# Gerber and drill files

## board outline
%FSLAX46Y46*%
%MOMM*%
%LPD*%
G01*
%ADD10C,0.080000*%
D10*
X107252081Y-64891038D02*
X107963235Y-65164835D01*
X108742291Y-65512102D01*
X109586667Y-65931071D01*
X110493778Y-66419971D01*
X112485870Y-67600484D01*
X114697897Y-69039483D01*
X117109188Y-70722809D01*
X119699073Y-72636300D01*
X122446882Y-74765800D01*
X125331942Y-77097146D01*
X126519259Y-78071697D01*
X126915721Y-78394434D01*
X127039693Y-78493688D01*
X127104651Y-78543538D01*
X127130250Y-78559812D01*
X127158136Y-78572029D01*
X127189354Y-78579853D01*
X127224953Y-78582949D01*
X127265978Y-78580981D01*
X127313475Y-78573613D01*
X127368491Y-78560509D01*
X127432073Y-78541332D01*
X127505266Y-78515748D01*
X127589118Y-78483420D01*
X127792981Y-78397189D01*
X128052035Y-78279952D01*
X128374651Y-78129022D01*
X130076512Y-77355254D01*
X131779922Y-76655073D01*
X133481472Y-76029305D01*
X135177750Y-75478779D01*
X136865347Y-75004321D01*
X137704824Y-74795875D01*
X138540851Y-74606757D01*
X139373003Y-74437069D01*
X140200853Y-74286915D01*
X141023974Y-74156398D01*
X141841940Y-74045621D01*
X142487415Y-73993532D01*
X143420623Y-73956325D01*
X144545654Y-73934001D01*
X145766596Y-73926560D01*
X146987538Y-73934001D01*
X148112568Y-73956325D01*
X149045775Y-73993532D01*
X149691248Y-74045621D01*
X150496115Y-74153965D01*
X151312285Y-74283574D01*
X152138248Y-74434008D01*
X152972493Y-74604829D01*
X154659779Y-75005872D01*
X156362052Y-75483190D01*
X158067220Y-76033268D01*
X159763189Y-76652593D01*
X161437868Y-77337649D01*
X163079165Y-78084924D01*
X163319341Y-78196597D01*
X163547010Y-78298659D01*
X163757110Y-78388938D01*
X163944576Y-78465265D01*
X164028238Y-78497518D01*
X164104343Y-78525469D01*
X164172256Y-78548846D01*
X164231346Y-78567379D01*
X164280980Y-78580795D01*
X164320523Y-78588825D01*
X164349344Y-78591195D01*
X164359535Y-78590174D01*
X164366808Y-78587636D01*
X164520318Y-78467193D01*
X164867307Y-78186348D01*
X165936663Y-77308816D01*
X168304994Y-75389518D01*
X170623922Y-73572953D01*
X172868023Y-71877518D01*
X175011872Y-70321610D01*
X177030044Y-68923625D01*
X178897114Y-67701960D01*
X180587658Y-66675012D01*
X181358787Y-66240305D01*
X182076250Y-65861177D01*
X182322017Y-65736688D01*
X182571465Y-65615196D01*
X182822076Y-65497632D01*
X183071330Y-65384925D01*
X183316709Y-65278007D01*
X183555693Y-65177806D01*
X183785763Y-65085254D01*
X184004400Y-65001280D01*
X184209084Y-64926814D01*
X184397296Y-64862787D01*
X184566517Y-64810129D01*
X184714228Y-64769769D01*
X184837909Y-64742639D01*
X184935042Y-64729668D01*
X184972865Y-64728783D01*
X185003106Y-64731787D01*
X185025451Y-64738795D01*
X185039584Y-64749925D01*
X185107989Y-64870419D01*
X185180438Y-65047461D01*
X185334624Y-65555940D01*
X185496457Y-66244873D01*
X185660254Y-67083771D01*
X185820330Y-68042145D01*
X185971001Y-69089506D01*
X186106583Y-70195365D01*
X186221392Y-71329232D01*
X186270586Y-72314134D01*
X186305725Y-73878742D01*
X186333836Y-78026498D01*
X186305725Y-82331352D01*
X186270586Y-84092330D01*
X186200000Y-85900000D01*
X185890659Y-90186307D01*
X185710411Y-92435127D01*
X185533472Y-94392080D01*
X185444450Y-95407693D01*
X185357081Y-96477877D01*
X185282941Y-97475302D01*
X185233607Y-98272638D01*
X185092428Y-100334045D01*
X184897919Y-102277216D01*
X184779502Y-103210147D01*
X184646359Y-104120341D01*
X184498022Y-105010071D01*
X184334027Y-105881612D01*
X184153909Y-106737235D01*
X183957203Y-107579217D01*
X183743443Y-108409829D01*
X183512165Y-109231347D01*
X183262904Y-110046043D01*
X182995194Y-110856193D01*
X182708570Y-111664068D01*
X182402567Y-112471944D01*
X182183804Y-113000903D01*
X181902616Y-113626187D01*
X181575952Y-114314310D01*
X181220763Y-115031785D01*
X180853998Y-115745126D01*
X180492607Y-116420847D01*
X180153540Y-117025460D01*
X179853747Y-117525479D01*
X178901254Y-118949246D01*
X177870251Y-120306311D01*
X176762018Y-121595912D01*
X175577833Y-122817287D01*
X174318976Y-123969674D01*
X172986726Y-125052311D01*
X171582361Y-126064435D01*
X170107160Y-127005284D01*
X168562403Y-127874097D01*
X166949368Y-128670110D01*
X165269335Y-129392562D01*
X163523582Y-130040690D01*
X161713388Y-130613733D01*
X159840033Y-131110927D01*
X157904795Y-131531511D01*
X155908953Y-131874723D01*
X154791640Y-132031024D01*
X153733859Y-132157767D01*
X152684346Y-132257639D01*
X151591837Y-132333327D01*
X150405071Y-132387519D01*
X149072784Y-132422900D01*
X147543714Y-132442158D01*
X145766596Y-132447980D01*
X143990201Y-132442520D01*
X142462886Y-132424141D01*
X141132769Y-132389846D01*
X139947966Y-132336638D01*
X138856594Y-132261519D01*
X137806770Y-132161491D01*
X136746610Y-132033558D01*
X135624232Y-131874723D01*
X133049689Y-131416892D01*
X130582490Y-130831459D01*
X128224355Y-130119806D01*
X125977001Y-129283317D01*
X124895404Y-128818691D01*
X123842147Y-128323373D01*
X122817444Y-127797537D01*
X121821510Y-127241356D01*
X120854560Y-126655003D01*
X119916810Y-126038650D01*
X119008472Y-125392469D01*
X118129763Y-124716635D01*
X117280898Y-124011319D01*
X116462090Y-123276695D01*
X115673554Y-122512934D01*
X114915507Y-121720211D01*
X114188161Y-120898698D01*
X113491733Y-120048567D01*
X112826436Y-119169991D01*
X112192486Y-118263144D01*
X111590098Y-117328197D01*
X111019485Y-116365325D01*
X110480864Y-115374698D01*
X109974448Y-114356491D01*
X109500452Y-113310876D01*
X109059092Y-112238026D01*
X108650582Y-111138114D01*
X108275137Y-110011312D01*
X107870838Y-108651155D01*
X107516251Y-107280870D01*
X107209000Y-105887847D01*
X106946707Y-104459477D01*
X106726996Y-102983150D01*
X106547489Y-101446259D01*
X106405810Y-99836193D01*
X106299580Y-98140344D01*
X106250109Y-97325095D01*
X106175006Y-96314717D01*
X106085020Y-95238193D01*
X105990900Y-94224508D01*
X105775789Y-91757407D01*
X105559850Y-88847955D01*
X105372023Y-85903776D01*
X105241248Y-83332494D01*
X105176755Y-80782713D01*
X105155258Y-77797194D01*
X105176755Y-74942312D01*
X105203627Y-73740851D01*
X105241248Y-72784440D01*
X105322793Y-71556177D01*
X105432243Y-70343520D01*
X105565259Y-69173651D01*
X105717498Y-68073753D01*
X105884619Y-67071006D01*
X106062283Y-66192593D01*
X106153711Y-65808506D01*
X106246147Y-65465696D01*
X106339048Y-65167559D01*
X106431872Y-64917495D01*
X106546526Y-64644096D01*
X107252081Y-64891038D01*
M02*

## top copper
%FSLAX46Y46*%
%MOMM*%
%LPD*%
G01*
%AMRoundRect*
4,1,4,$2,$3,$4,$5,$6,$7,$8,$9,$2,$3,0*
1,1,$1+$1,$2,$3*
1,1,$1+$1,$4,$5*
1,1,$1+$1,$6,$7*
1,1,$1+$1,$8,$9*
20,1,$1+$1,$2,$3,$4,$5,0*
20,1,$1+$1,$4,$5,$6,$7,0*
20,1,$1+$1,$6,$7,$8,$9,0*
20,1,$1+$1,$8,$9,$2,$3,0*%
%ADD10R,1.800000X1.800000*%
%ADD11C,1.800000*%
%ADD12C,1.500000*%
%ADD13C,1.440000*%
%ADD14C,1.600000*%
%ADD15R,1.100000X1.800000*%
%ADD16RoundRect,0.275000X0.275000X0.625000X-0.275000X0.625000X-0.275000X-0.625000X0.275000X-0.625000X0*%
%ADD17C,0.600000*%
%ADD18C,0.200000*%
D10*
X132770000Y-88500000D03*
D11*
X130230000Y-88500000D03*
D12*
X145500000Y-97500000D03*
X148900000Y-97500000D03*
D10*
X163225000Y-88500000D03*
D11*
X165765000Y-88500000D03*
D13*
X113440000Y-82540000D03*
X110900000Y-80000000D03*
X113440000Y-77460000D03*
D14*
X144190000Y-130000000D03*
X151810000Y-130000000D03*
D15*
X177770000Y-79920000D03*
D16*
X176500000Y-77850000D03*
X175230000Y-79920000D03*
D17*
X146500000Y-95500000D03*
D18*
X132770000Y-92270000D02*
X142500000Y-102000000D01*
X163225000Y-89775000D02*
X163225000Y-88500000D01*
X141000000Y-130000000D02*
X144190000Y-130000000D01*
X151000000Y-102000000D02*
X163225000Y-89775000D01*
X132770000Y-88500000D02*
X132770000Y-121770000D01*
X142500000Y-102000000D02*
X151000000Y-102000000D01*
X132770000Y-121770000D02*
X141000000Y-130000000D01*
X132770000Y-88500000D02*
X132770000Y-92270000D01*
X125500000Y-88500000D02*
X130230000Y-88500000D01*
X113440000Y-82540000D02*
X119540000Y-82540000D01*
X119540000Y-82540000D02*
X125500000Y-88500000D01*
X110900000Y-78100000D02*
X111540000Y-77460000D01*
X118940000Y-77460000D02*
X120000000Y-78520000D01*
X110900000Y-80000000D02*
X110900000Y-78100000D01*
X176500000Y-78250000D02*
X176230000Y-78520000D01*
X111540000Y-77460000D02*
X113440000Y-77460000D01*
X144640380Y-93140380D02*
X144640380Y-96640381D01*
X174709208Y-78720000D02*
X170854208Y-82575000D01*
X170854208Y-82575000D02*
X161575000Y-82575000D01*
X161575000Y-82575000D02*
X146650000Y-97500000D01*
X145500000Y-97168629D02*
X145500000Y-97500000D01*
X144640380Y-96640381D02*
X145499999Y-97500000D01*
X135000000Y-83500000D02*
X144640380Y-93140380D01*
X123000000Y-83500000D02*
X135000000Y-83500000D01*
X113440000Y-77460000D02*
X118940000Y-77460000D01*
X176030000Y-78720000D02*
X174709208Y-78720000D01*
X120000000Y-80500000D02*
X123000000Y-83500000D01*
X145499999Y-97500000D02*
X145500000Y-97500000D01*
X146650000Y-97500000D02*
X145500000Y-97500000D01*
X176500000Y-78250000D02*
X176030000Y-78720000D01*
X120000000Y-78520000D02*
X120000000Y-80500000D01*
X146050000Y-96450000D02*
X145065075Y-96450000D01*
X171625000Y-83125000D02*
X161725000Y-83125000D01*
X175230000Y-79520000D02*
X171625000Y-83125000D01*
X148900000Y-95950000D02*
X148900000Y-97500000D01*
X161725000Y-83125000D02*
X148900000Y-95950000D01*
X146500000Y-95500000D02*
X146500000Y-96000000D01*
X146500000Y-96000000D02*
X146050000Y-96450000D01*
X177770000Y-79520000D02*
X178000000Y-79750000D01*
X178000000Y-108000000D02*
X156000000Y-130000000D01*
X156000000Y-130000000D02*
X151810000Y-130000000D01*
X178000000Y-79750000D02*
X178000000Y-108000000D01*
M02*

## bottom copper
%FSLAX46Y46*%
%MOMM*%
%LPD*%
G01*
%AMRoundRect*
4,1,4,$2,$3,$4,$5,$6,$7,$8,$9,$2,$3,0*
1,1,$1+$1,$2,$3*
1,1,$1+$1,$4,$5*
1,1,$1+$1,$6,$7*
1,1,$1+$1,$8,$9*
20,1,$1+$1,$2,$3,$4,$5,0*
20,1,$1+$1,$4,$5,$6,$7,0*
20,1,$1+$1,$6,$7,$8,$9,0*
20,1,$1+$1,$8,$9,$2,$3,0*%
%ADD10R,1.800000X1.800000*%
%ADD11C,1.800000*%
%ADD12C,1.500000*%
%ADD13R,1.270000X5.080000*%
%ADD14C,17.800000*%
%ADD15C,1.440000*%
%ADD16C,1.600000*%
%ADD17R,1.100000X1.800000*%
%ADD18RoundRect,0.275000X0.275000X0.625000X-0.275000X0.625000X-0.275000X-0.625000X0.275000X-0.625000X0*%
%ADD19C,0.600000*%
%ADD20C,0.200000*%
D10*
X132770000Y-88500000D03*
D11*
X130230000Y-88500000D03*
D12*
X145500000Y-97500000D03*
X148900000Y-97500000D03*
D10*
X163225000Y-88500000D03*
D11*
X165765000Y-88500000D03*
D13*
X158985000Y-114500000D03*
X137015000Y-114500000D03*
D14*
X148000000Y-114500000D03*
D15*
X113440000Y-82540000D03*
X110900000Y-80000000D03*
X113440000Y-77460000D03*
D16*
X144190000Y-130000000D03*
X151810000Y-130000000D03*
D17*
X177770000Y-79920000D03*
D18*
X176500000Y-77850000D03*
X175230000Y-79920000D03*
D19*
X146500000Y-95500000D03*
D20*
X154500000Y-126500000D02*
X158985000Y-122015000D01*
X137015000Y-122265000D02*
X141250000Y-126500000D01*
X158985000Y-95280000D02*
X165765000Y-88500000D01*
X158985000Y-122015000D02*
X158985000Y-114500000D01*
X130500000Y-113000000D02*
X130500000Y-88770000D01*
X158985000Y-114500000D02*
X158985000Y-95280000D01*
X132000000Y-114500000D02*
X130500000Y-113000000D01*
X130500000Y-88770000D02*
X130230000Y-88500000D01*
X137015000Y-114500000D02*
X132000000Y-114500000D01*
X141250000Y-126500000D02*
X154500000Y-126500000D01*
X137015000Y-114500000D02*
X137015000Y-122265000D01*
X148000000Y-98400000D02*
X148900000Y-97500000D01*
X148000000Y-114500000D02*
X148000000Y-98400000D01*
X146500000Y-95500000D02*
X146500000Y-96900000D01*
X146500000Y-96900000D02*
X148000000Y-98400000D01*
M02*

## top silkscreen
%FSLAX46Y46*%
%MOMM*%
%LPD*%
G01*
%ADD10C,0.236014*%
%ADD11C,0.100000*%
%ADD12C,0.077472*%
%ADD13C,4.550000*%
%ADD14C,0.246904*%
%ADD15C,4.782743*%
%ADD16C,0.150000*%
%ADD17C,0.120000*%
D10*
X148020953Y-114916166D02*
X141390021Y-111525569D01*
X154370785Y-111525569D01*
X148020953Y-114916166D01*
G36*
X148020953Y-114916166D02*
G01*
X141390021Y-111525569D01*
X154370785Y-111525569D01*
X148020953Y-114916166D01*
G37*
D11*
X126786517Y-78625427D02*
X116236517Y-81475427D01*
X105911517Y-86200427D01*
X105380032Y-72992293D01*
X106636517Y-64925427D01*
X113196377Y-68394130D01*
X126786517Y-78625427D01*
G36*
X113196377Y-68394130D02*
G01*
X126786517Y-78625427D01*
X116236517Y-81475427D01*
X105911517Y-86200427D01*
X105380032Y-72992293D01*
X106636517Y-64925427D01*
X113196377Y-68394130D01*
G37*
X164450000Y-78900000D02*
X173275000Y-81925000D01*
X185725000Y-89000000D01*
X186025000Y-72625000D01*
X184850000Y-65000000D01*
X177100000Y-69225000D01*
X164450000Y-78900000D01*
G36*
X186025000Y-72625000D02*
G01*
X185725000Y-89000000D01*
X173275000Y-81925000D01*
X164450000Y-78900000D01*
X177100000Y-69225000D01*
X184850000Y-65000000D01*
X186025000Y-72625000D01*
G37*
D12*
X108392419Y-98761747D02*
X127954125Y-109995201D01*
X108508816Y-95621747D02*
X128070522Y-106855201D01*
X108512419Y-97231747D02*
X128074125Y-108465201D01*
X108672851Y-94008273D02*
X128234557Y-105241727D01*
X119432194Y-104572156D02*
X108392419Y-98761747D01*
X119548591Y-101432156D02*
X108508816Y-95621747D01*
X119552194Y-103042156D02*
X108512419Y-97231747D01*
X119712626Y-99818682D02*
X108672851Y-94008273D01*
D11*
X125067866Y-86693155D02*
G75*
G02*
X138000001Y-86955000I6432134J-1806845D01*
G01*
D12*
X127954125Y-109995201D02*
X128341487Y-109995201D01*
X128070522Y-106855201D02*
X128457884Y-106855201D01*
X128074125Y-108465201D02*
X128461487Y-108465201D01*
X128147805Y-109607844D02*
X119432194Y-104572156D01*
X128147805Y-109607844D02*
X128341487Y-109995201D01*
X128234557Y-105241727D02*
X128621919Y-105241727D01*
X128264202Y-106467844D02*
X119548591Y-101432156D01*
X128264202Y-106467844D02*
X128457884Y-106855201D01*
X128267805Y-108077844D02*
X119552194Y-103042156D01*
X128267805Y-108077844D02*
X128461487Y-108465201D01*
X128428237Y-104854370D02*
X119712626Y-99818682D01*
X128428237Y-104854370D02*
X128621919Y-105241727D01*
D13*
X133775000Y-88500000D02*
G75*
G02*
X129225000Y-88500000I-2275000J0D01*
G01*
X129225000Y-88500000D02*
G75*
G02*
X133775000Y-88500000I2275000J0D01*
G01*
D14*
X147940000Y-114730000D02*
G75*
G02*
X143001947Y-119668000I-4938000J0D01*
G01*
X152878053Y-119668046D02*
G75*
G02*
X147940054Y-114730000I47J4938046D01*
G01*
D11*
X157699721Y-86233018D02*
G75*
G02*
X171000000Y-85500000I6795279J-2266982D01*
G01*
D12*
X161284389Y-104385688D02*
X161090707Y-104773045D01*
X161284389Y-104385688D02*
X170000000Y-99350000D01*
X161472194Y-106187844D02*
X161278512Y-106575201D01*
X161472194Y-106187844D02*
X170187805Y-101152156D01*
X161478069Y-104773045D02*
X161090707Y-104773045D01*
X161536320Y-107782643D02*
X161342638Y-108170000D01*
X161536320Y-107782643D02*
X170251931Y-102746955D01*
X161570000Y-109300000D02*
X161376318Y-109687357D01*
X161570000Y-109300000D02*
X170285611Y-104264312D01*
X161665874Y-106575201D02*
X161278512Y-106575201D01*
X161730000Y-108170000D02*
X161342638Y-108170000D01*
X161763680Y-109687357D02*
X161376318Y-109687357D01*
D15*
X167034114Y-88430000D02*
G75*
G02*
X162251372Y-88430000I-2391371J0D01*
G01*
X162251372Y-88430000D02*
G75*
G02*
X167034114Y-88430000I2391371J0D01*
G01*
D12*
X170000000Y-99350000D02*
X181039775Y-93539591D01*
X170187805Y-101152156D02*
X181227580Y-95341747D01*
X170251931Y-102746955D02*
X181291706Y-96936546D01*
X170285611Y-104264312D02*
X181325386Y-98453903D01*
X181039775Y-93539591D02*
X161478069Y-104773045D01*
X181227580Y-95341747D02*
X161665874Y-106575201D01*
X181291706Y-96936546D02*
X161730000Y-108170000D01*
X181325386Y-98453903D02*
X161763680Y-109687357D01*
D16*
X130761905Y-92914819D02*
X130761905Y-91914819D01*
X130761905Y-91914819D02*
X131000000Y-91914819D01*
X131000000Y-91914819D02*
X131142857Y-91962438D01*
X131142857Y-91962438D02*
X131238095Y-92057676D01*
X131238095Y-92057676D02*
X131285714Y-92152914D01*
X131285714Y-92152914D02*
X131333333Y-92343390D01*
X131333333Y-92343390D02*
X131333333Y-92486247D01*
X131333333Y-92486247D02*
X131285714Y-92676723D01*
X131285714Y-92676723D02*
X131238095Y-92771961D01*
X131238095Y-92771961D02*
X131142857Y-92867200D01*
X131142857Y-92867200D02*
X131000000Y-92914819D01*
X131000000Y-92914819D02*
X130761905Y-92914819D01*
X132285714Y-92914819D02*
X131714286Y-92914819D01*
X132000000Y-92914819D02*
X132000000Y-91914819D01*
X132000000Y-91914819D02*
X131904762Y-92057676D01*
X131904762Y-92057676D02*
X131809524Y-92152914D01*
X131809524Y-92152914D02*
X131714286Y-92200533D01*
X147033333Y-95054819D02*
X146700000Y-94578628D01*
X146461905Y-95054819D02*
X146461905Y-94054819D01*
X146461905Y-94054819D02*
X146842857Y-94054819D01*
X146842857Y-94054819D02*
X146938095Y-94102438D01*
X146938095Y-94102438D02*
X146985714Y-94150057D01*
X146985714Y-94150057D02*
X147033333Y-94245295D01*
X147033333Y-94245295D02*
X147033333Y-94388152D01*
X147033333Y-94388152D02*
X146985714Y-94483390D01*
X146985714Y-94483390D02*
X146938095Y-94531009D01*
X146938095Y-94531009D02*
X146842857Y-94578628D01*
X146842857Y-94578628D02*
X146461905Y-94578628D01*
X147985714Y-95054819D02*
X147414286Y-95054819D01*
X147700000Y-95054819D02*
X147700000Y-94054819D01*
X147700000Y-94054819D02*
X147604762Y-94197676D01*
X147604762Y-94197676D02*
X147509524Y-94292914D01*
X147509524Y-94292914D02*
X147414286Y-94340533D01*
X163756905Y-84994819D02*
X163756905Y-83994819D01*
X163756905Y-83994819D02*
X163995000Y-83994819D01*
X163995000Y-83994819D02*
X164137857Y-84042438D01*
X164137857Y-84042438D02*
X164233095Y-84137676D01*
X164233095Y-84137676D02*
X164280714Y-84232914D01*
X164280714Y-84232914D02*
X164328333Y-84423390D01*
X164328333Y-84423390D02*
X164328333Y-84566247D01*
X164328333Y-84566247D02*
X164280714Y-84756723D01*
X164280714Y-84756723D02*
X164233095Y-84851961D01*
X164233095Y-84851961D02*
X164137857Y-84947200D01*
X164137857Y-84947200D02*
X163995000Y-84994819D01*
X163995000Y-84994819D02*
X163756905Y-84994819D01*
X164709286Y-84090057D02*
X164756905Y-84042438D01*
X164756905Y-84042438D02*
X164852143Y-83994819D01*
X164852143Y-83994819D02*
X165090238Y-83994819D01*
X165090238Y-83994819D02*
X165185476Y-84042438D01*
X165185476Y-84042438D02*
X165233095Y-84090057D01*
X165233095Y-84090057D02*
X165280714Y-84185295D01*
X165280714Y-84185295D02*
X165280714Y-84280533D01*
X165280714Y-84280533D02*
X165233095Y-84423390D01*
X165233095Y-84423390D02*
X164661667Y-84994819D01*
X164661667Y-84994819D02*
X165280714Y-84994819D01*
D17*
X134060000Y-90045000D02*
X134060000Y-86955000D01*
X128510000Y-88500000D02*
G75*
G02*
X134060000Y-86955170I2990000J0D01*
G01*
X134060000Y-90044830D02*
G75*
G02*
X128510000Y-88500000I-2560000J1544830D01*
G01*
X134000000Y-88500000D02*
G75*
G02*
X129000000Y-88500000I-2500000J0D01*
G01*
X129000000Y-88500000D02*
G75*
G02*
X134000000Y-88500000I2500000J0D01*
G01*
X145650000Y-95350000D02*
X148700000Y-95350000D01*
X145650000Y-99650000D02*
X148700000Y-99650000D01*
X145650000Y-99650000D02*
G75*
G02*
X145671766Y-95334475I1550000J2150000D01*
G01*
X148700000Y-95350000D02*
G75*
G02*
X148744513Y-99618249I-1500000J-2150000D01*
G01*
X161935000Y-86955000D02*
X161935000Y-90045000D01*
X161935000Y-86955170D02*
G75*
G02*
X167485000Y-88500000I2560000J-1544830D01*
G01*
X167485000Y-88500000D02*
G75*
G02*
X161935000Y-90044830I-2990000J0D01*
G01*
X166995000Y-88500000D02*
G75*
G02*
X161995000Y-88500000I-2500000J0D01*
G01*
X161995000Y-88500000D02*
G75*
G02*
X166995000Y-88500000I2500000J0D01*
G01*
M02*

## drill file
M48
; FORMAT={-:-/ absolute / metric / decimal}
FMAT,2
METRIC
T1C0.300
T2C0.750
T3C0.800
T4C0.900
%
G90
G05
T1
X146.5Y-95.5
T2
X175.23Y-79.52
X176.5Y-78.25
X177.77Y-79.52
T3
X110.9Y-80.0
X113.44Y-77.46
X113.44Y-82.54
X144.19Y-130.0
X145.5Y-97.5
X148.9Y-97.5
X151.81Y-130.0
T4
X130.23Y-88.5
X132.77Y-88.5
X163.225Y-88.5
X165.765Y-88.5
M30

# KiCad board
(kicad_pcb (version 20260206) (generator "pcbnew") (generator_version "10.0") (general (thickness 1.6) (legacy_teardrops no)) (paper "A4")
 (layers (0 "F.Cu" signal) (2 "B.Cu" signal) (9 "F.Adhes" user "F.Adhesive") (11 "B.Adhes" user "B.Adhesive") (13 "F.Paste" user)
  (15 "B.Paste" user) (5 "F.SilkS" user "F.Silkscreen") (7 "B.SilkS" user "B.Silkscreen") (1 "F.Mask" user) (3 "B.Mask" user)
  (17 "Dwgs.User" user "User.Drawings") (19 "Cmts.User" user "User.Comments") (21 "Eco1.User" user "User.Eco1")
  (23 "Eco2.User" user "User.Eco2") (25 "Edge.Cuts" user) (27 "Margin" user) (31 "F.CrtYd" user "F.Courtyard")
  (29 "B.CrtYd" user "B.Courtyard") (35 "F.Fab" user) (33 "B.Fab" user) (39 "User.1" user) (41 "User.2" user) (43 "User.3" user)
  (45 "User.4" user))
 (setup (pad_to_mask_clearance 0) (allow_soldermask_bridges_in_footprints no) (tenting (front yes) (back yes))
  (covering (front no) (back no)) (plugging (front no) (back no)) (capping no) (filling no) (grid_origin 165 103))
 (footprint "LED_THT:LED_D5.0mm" (layer "F.Cu") (at 132.77 88.5 180)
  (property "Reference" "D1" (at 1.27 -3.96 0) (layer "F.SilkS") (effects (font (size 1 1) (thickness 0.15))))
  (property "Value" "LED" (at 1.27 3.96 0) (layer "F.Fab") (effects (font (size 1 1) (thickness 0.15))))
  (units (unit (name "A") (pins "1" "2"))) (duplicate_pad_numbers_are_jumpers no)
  (fp_line (start -1.29 -1.545) (end -1.29 1.545) (stroke (width 0.12) (type solid)) (layer "F.SilkS"))
  (fp_arc (start 4.26 0) (mid 2.071779 2.880495) (end -1.29 1.54483) (stroke (width 0.12) (type solid)) (layer "F.SilkS"))
  (fp_arc (start -1.29 -1.54483) (mid 2.071779 -2.880495) (end 4.26 0) (stroke (width 0.12) (type solid)) (layer "F.SilkS"))
  (fp_circle (center 1.27 0) (end 3.77 0) (stroke (width 0.12) (type solid)) (fill no) (layer "F.SilkS"))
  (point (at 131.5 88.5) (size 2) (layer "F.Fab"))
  (pad "1" thru_hole rect (at 0 0 180) (size 1.8 1.8) (drill 0.9) (layers "*.Cu" "*.Mask") (remove_unused_layers no) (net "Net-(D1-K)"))
  (pad "2" thru_hole circle (at 2.54 0 180) (size 1.8 1.8) (drill 0.9) (layers "*.Cu" "*.Mask") (remove_unused_layers no)
   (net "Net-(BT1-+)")))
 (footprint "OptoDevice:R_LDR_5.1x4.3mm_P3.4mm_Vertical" (layer "F.Cu") (at 145.5 97.5)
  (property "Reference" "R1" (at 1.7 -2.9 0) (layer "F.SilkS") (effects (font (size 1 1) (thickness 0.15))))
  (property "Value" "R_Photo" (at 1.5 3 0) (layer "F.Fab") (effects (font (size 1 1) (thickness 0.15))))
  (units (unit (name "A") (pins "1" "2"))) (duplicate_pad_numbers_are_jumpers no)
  (fp_line (start 0.15 -2.15) (end 3.2 -2.15) (stroke (width 0.12) (type solid)) (layer "F.SilkS"))
  (fp_line (start 0.15 2.15) (end 3.2 2.15) (stroke (width 0.12) (type solid)) (layer "F.SilkS"))
  (fp_arc (start 0.15 2.15) (mid -0.950438 -0.013368) (end 0.171766 -2.165525) (stroke (width 0.12) (type solid)) (layer "F.SilkS"))
  (fp_arc (start 3.2 -2.15) (mid 4.321403 -0.027338) (end 3.244513 2.118249) (stroke (width 0.12) (type solid)) (layer "F.SilkS"))
  (pad "1" thru_hole circle (at 0 0) (size 1.5 1.5) (drill 0.8) (layers "*.Cu" "*.Mask") (remove_unused_layers no) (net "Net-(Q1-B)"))
  (pad "2" thru_hole circle (at 3.4 0) (size 1.5 1.5) (drill 0.8) (layers "*.Cu" "*.Mask") (remove_unused_layers no) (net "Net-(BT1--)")))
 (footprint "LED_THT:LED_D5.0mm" (layer "F.Cu") (at 163.225 88.5)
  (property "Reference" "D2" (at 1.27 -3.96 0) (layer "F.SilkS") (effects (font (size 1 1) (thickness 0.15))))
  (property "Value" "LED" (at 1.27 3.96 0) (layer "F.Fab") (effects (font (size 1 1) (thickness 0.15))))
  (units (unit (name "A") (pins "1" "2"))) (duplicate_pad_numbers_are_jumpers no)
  (fp_line (start -1.29 -1.545) (end -1.29 1.545) (stroke (width 0.12) (type solid)) (layer "F.SilkS"))
  (fp_arc (start -1.29 -1.54483) (mid 2.071779 -2.880495) (end 4.26 0) (stroke (width 0.12) (type solid)) (layer "F.SilkS"))
  (fp_arc (start 4.26 0) (mid 2.071779 2.880495) (end -1.29 1.54483) (stroke (width 0.12) (type solid)) (layer "F.SilkS"))
  (fp_circle (center 1.27 0) (end 3.77 0) (stroke (width 0.12) (type solid)) (fill no) (layer "F.SilkS"))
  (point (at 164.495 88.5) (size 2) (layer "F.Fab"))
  (pad "1" thru_hole rect (at 0 0) (size 1.8 1.8) (drill 0.9) (layers "*.Cu" "*.Mask") (remove_unused_layers no) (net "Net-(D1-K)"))
  (pad "2" thru_hole circle (at 2.54 0) (size 1.8 1.8) (drill 0.9) (layers "*.Cu" "*.Mask") (remove_unused_layers no) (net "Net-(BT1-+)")))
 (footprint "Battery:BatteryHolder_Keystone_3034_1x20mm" (layer "B.Cu") (at 148 114.5 180)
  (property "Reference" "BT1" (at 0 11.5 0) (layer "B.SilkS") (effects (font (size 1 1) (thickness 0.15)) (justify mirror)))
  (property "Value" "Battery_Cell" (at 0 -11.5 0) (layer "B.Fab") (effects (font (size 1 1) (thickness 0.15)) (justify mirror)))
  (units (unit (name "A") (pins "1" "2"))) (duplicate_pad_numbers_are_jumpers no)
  (pad "1" smd rect (at -10.985 0 180) (size 1.27 5.08) (layers "B.Cu" "B.Mask" "B.Paste") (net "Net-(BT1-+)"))
  (pad "1" smd rect (at 10.985 0 180) (size 1.27 5.08) (layers "B.Cu" "B.Mask" "B.Paste") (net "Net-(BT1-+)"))
  (pad "2" smd circle (at 0 0 180) (size 17.8 17.8) (layers "B.Cu" "B.Mask") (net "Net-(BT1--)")))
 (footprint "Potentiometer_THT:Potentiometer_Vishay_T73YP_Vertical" (layer "B.Cu") (at 113.44 82.54 180)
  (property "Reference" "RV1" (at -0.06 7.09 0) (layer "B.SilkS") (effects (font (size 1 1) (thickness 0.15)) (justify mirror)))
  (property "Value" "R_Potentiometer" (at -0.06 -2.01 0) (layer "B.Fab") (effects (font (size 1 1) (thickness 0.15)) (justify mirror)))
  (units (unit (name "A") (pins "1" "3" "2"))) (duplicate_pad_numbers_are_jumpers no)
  (pad "1" thru_hole circle (at 0 0 180) (size 1.44 1.44) (drill 0.8) (layers "*.Cu" "*.Mask") (remove_unused_layers no) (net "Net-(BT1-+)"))
  (pad "2" thru_hole circle (at 2.54 2.54 180) (size 1.44 1.44) (drill 0.8) (layers "*.Cu" "*.Mask") (remove_unused_layers no)
   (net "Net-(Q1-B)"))
  (pad "3" thru_hole circle (at 0 5.08 180) (size 1.44 1.44) (drill 0.8) (layers "*.Cu" "*.Mask") (remove_unused_layers no)
   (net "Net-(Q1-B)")))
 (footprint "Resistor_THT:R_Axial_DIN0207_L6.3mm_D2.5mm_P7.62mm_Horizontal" (layer "B.Cu") (at 144.19 130)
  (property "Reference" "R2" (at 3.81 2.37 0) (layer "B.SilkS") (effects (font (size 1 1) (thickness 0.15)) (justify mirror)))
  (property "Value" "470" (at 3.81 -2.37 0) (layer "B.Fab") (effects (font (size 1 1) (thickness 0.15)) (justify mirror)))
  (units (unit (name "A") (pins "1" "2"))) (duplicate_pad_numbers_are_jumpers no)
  (pad "1" thru_hole circle (at 0 0) (size 1.6 1.6) (drill 0.8) (layers "*.Cu" "*.Mask") (remove_unused_layers no) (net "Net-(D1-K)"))
  (pad "2" thru_hole circle (at 7.62 0) (size 1.6 1.6) (drill 0.8) (layers "*.Cu" "*.Mask") (remove_unused_layers no) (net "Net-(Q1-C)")))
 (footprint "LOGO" (layer "B.Cu") (at 124.781072 101.737915 180)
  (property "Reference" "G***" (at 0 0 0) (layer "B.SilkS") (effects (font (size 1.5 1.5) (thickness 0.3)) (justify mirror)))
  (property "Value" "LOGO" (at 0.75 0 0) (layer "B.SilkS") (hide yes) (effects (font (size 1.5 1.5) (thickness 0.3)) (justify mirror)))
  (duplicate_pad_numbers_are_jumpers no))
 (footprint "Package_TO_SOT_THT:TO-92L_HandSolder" (layer "B.Cu") (at 177.77 79.52 180)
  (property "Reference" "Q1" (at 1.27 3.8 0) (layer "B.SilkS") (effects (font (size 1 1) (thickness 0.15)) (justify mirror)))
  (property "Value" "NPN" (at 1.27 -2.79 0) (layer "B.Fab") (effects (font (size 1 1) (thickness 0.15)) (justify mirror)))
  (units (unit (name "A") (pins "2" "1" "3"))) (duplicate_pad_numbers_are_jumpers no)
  (pad "1" thru_hole rect (at 0 0 180) (size 1.1 1.8) (drill 0.75 (offset 0 -0.4)) (layers "*.Cu" "*.Mask") (remove_unused_layers no)
   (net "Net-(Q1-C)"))
  (pad "2" thru_hole roundrect (at 1.27 1.27 180) (size 1.1 1.8) (drill 0.75 (offset 0 0.4)) (layers "*.Cu" "*.Mask")
   (remove_unused_layers no) (roundrect_rratio 0.25) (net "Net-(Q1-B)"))
  (pad "3" thru_hole roundrect (at 2.54 0 180) (size 1.1 1.8) (drill 0.75 (offset 0 -0.4)) (layers "*.Cu" "*.Mask")
   (remove_unused_layers no) (roundrect_rratio 0.25) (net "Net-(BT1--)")))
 (gr_poly
  (pts (xy 148.020953 114.916166) (xy 141.390021 111.525569) (xy 154.370785 111.525569)) (stroke (width 0.236014) (type solid)) (fill yes)
  (layer "F.SilkS"))
 (gr_poly
  (pts (xy 126.786517 78.625427) (xy 116.236517 81.475427) (xy 105.911517 86.200427) (xy 105.380032 72.992293) (xy 106.636517 64.925427)
   (xy 113.196377 68.39413))
  (stroke (width 0.1) (type solid)) (fill yes) (layer "F.SilkS"))
 (gr_poly
  (pts (xy 164.45 78.9) (xy 173.275 81.925) (xy 185.725 89) (xy 186.025 72.625) (xy 184.85 65) (xy 177.1 69.225))
  (stroke (width 0.1) (type solid)) (fill yes) (layer "F.SilkS"))
 (gr_line (start 108.392419 98.761747) (end 127.954125 109.995201) (stroke (width 0.077472) (type default)) (layer "F.SilkS"))
 (gr_line (start 108.508816 95.621747) (end 128.070522 106.855201) (stroke (width 0.077472) (type default)) (layer "F.SilkS"))
 (gr_line (start 108.512419 97.231747) (end 128.074125 108.465201) (stroke (width 0.077472) (type default)) (layer "F.SilkS"))
 (gr_line (start 108.672851 94.008273) (end 128.234557 105.241727) (stroke (width 0.077472) (type default)) (layer "F.SilkS"))
 (gr_line (start 119.432194 104.572156) (end 108.392419 98.761747) (stroke (width 0.077472) (type default)) (layer "F.SilkS"))
 (gr_line (start 119.548591 101.432156) (end 108.508816 95.621747) (stroke (width 0.077472) (type default)) (layer "F.SilkS"))
 (gr_line (start 119.552194 103.042156) (end 108.512419 97.231747) (stroke (width 0.077472) (type default)) (layer "F.SilkS"))
 (gr_line (start 119.712626 99.818682) (end 108.672851 94.008273) (stroke (width 0.077472) (type default)) (layer "F.SilkS"))
 (gr_arc (start 125.067866 86.693155) (mid 131.635248 81.820274) (end 138 86.955) (stroke (width 0.1) (type default)) (layer "F.SilkS"))
 (gr_line (start 127.954125 109.995201) (end 128.341487 109.995201) (stroke (width 0.077472) (type default)) (layer "F.SilkS"))
 (gr_line (start 128.070522 106.855201) (end 128.457884 106.855201) (stroke (width 0.077472) (type default)) (layer "F.SilkS"))
 (gr_line (start 128.074125 108.465201) (end 128.461487 108.465201) (stroke (width 0.077472) (type default)) (layer "F.SilkS"))
 (gr_line (start 128.147805 109.607844) (end 119.432194 104.572156) (stroke (width 0.077472) (type default)) (layer "F.SilkS"))
 (gr_line (start 128.147805 109.607844) (end 128.341487 109.995201) (stroke (width 0.077472) (type default)) (layer "F.SilkS"))
 (gr_line (start 128.234557 105.241727) (end 128.621919 105.241727) (stroke (width 0.077472) (type default)) (layer "F.SilkS"))
 (gr_line (start 128.264202 106.467844) (end 119.548591 101.432156) (stroke (width 0.077472) (type default)) (layer "F.SilkS"))
 (gr_line (start 128.264202 106.467844) (end 128.457884 106.855201) (stroke (width 0.077472) (type default)) (layer "F.SilkS"))
 (gr_line (start 128.267805 108.077844) (end 119.552194 103.042156) (stroke (width 0.077472) (type default)) (layer "F.SilkS"))
 (gr_line (start 128.267805 108.077844) (end 128.461487 108.465201) (stroke (width 0.077472) (type default)) (layer "F.SilkS"))
 (gr_line (start 128.428237 104.85437) (end 119.712626 99.818682) (stroke (width 0.077472) (type default)) (layer "F.SilkS"))
 (gr_line (start 128.428237 104.85437) (end 128.621919 105.241727) (stroke (width 0.077472) (type default)) (layer "F.SilkS"))
 (gr_circle (center 131.5 88.5) (end 136 88.5) (stroke (width 0.1) (type solid)) (fill yes) (layer "F.SilkS"))
 (gr_arc (start 147.94 114.73) (mid 146.493678 118.221731) (end 143.001947 119.668046) (stroke (width 0.246904) (type default))
  (layer "F.SilkS"))
 (gr_arc (start 152.878053 119.668046) (mid 149.386325 118.221727) (end 147.94 114.73) (stroke (width 0.246904) (type default))
  (layer "F.SilkS"))
 (gr_arc (start 157.699721 86.233018) (mid 164.100799 81.347404) (end 171 85.5) (stroke (width 0.1) (type default)) (layer "F.SilkS"))
 (gr_line (start 161.284389 104.385688) (end 161.090707 104.773045) (stroke (width 0.077472) (type default)) (layer "F.SilkS"))
 (gr_line (start 161.284389 104.385688) (end 170 99.35) (stroke (width 0.077472) (type default)) (layer "F.SilkS"))
 (gr_line (start 161.472194 106.187844) (end 161.278512 106.575201) (stroke (width 0.077472) (type default)) (layer "F.SilkS"))
 (gr_line (start 161.472194 106.187844) (end 170.187805 101.152156) (stroke (width 0.077472) (type default)) (layer "F.SilkS"))
 (gr_line (start 161.478069 104.773045) (end 161.090707 104.773045) (stroke (width 0.077472) (type default)) (layer "F.SilkS"))
 (gr_line (start 161.53632 107.782643) (end 161.342638 108.17) (stroke (width 0.077472) (type default)) (layer "F.SilkS"))
 (gr_line (start 161.53632 107.782643) (end 170.251931 102.746955) (stroke (width 0.077472) (type default)) (layer "F.SilkS"))
 (gr_line (start 161.57 109.3) (end 161.376318 109.687357) (stroke (width 0.077472) (type default)) (layer "F.SilkS"))
 (gr_line (start 161.57 109.3) (end 170.285611 104.264312) (stroke (width 0.077472) (type default)) (layer "F.SilkS"))
 (gr_line (start 161.665874 106.575201) (end 161.278512 106.575201) (stroke (width 0.077472) (type default)) (layer "F.SilkS"))
 (gr_line (start 161.73 108.17) (end 161.342638 108.17) (stroke (width 0.077472) (type default)) (layer "F.SilkS"))
 (gr_line (start 161.76368 109.687357) (end 161.376318 109.687357) (stroke (width 0.077472) (type default)) (layer "F.SilkS"))
 (gr_circle (center 164.642743 88.43) (end 169.349 88.93) (stroke (width 0.1) (type solid)) (fill yes) (layer "F.SilkS"))
 (gr_line (start 170 99.35) (end 181.039775 93.539591) (stroke (width 0.077472) (type default)) (layer "F.SilkS"))
 (gr_line (start 170.187805 101.152156) (end 181.22758 95.341747) (stroke (width 0.077472) (type default)) (layer "F.SilkS"))
 (gr_line (start 170.251931 102.746955) (end 181.291706 96.936546) (stroke (width 0.077472) (type default)) (layer "F.SilkS"))
 (gr_line (start 170.285611 104.264312) (end 181.325386 98.453903) (stroke (width 0.077472) (type default)) (layer "F.SilkS"))
 (gr_line (start 181.039775 93.539591) (end 161.478069 104.773045) (stroke (width 0.077472) (type default)) (layer "F.SilkS"))
 (gr_line (start 181.22758 95.341747) (end 161.665874 106.575201) (stroke (width 0.077472) (type default)) (layer "F.SilkS"))
 (gr_line (start 181.291706 96.936546) (end 161.73 108.17) (stroke (width 0.077472) (type default)) (layer "F.SilkS"))
 (gr_line (start 181.325386 98.453903) (end 161.76368 109.687357) (stroke (width 0.077472) (type default)) (layer "F.SilkS"))
 (gr_poly
  (pts (xy 107.252081 64.891038) (xy 107.963235 65.164835) (xy 108.742291 65.512102) (xy 109.586667 65.931071) (xy 110.493778 66.419971)
   (xy 112.48587 67.600484) (xy 114.697897 69.039483) (xy 117.109188 70.722809) (xy 119.699073 72.6363) (xy 122.446882 74.7658)
   (xy 125.331942 77.097146) (xy 126.519259 78.071697) (xy 126.915721 78.394434) (xy 127.039693 78.493688) (xy 127.104651 78.543538)
   (xy 127.13025 78.559812) (xy 127.158136 78.572029) (xy 127.189354 78.579853) (xy 127.224953 78.582949) (xy 127.265978 78.580981)
   (xy 127.313475 78.573613) (xy 127.368491 78.560509) (xy 127.432073 78.541332) (xy 127.505266 78.515748) (xy 127.589118 78.48342)
   (xy 127.792981 78.397189) (xy 128.052035 78.279952) (xy 128.374651 78.129022) (xy 130.076512 77.355254) (xy 131.779922 76.655073)
   (xy 133.481472 76.029305) (xy 135.17775 75.478779) (xy 136.865347 75.004321) (xy 137.704824 74.795875) (xy 138.540851 74.606757)
   (xy 139.373003 74.437069) (xy 140.200853 74.286915) (xy 141.023974 74.156398) (xy 141.84194 74.045621) (xy 142.487415 73.993532)
   (xy 143.420623 73.956325) (xy 144.545654 73.934001) (xy 145.766596 73.92656) (xy 146.987538 73.934001) (xy 148.112568 73.956325)
   (xy 149.045775 73.993532) (xy 149.691248 74.045621) (xy 150.496115 74.153965) (xy 151.312285 74.283574) (xy 152.138248 74.434008)
   (xy 152.972493 74.604829) (xy 154.659779 75.005872) (xy 156.362052 75.48319) (xy 158.06722 76.033268) (xy 159.763189 76.652593)
   (xy 161.437868 77.337649) (xy 163.079165 78.084924) (xy 163.319341 78.196597) (xy 163.54701 78.298659) (xy 163.75711 78.388938)
   (xy 163.944576 78.465265) (xy 164.028238 78.497518) (xy 164.104343 78.525469) (xy 164.172256 78.548846) (xy 164.231346 78.567379)
   (xy 164.28098 78.580795) (xy 164.320523 78.588825) (xy 164.349344 78.591195) (xy 164.359535 78.590174) (xy 164.366808 78.587636)
   (xy 164.520318 78.467193) (xy 164.867307 78.186348) (xy 165.936663 77.308816) (xy 168.304994 75.389518) (xy 170.623922 73.572953)
   (xy 172.868023 71.877518) (xy 175.011872 70.32161) (xy 177.030044 68.923625) (xy 178.897114 67.70196) (xy 180.587658 66.675012)
   (xy 181.358787 66.240305) (xy 182.07625 65.861177) (xy 182.322017 65.736688) (xy 182.571465 65.615196) (xy 182.822076 65.497632)
   (xy 183.07133 65.384925) (xy 183.316709 65.278007) (xy 183.555693 65.177806) (xy 183.785763 65.085254) (xy 184.0044 65.00128)
   (xy 184.209084 64.926814) (xy 184.397296 64.862787) (xy 184.566517 64.810129) (xy 184.714228 64.769769) (xy 184.837909 64.742639)
   (xy 184.935042 64.729668) (xy 184.972865 64.728783) (xy 185.003106 64.731787) (xy 185.025451 64.738795) (xy 185.039584 64.749925)
   (xy 185.107989 64.870419) (xy 185.180438 65.047461) (xy 185.334624 65.55594) (xy 185.496457 66.244873) (xy 185.660254 67.083771)
   (xy 185.82033 68.042145) (xy 185.971001 69.089506) (xy 186.106583 70.195365) (xy 186.221392 71.329232) (xy 186.270586 72.314134)
   (xy 186.305725 73.878742) (xy 186.333836 78.026498) (xy 186.305725 82.331352) (xy 186.270586 84.09233) (xy 186.2 85.9)
   (xy 185.890659 90.186307) (xy 185.710411 92.435127) (xy 185.533472 94.39208) (xy 185.44445 95.407693) (xy 185.357081 96.477877)
   (xy 185.282941 97.475302) (xy 185.233607 98.272638) (xy 185.092428 100.334045) (xy 184.897919 102.277216) (xy 184.779502 103.210147)
   (xy 184.646359 104.120341) (xy 184.498022 105.010071) (xy 184.334027 105.881612) (xy 184.153909 106.737235) (xy 183.957203 107.579217)
   (xy 183.743443 108.409829) (xy 183.512165 109.231347) (xy 183.262904 110.046043) (xy 182.995194 110.856193) (xy 182.70857 111.664068)
   (xy 182.402567 112.471944) (xy 182.183804 113.000903) (xy 181.902616 113.626187) (xy 181.575952 114.31431) (xy 181.220763 115.031785)
   (xy 180.853998 115.745126) (xy 180.492607 116.420847) (xy 180.15354 117.02546) (xy 179.853747 117.525479) (xy 178.901254 118.949246)
   (xy 177.870251 120.306311) (xy 176.762018 121.595912) (xy 175.577833 122.817287) (xy 174.318976 123.969674) (xy 172.986726 125.052311)
   (xy 171.582361 126.064435) (xy 170.10716 127.005284) (xy 168.562403 127.874097) (xy 166.949368 128.67011) (xy 165.269335 129.392562)
   (xy 163.523582 130.04069) (xy 161.713388 130.613733) (xy 159.840033 131.110927) (xy 157.904795 131.531511) (xy 155.908953 131.874723)
   (xy 154.79164 132.031024) (xy 153.733859 132.157767) (xy 152.684346 132.257639) (xy 151.591837 132.333327) (xy 150.405071 132.387519)
   (xy 149.072784 132.4229) (xy 147.543714 132.442158) (xy 145.766596 132.44798) (xy 143.990201 132.44252) (xy 142.462886 132.424141)
   (xy 141.132769 132.389846) (xy 139.947966 132.336638) (xy 138.856594 132.261519) (xy 137.80677 132.161491) (xy 136.74661 132.033558)
   (xy 135.624232 131.874723) (xy 133.049689 131.416892) (xy 130.58249 130.831459) (xy 128.224355 130.119806) (xy 125.977001 129.283317)
   (xy 124.895404 128.818691) (xy 123.842147 128.323373) (xy 122.817444 127.797537) (xy 121.82151 127.241356) (xy 120.85456 126.655003)
   (xy 119.91681 126.03865) (xy 119.008472 125.392469) (xy 118.129763 124.716635) (xy 117.280898 124.011319) (xy 116.46209 123.276695)
   (xy 115.673554 122.512934) (xy 114.915507 121.720211) (xy 114.188161 120.898698) (xy 113.491733 120.048567) (xy 112.826436 119.169991)
   (xy 112.192486 118.263144) (xy 111.590098 117.328197) (xy 111.019485 116.365325) (xy 110.480864 115.374698) (xy 109.974448 114.356491)
   (xy 109.500452 113.310876) (xy 109.059092 112.238026) (xy 108.650582 111.138114) (xy 108.275137 110.011312) (xy 107.870838 108.651155)
   (xy 107.516251 107.28087) (xy 107.209 105.887847) (xy 106.946707 104.459477) (xy 106.726996 102.98315) (xy 106.547489 101.446259)
   (xy 106.40581 99.836193) (xy 106.29958 98.140344) (xy 106.250109 97.325095) (xy 106.175006 96.314717) (xy 106.08502 95.238193)
   (xy 105.9909 94.224508) (xy 105.775789 91.757407) (xy 105.55985 88.847955) (xy 105.372023 85.903776) (xy 105.241248 83.332494)
   (xy 105.176755 80.782713) (xy 105.155258 77.797194) (xy 105.176755 74.942312) (xy 105.203627 73.740851) (xy 105.241248 72.78444)
   (xy 105.322793 71.556177) (xy 105.432243 70.34352) (xy 105.565259 69.173651) (xy 105.717498 68.073753) (xy 105.884619 67.071006)
   (xy 106.062283 66.192593) (xy 106.153711 65.808506) (xy 106.246147 65.465696) (xy 106.339048 65.167559) (xy 106.431872 64.917495)
   (xy 106.546526 64.644096))
  (stroke (width 0.08) (type solid)) (fill no) (layer "Edge.Cuts"))
 (segment (start 132.77 92.27) (end 142.5 102) (width 0.2) (layer "F.Cu") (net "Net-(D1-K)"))
 (segment (start 163.225 89.775) (end 163.225 88.5) (width 0.2) (layer "F.Cu") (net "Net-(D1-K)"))
 (segment (start 141 130) (end 144.19 130) (width 0.2) (layer "F.Cu") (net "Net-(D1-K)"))
 (segment (start 151 102) (end 163.225 89.775) (width 0.2) (layer "F.Cu") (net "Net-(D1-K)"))
 (segment (start 132.77 88.5) (end 132.77 121.77) (width 0.2) (layer "F.Cu") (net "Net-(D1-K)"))
 (segment (start 142.5 102) (end 151 102) (width 0.2) (layer "F.Cu") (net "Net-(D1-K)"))
 (segment (start 132.77 121.77) (end 141 130) (width 0.2) (layer "F.Cu") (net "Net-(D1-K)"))
 (segment (start 132.77 88.5) (end 132.77 92.27) (width 0.2) (layer "F.Cu") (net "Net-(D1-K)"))
 (segment (start 125.5 88.5) (end 130.23 88.5) (width 0.2) (layer "F.Cu") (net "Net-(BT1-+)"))
 (segment (start 113.44 82.54) (end 119.54 82.54) (width 0.2) (layer "F.Cu") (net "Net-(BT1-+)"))
 (segment (start 119.54 82.54) (end 125.5 88.5) (width 0.2) (layer "F.Cu") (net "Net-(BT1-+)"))
 (segment (start 154.5 126.5) (end 158.985 122.015) (width 0.2) (layer "B.Cu") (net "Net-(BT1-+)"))
 (segment (start 137.015 122.265) (end 141.25 126.5) (width 0.2) (layer "B.Cu") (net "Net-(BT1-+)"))
 (segment (start 158.985 95.28) (end 165.765 88.5) (width 0.2) (layer "B.Cu") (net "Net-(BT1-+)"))
 (segment (start 158.985 122.015) (end 158.985 114.5) (width 0.2) (layer "B.Cu") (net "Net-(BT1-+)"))
 (segment (start 130.5 113) (end 130.5 88.77) (width 0.2) (layer "B.Cu") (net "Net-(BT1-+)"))
 (segment (start 158.985 114.5) (end 158.985 95.28) (width 0.2) (layer "B.Cu") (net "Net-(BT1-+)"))
 (segment (start 132 114.5) (end 130.5 113) (width 0.2) (layer "B.Cu") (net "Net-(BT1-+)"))
 (segment (start 130.5 88.77) (end 130.23 88.5) (width 0.2) (layer "B.Cu") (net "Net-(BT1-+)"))
 (segment (start 137.015 114.5) (end 132 114.5) (width 0.2) (layer "B.Cu") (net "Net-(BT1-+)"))
 (segment (start 141.25 126.5) (end 154.5 126.5) (width 0.2) (layer "B.Cu") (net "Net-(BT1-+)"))
 (segment (start 137.015 114.5) (end 137.015 122.265) (width 0.2) (layer "B.Cu") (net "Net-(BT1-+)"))
 (segment (start 110.9 78.1) (end 111.54 77.46) (width 0.2) (layer "F.Cu") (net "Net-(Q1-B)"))
 (segment (start 118.94 77.46) (end 120 78.52) (width 0.2) (layer "F.Cu") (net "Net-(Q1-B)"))
 (segment (start 110.9 80) (end 110.9 78.1) (width 0.2) (layer "F.Cu") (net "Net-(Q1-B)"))
 (segment (start 176.5 78.25) (end 176.23 78.52) (width 0.2) (layer "F.Cu") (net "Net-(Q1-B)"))
 (segment (start 111.54 77.46) (end 113.44 77.46) (width 0.2) (layer "F.Cu") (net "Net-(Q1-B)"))
 (segment (start 144.64038 93.14038) (end 144.64038 96.640381) (width 0.2) (layer "F.Cu") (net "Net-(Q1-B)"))
 (segment (start 174.709208 78.72) (end 170.854208 82.575) (width 0.2) (layer "F.Cu") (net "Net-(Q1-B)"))
 (segment (start 170.854208 82.575) (end 161.575 82.575) (width 0.2) (layer "F.Cu") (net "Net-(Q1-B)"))
 (segment (start 161.575 82.575) (end 146.65 97.5) (width 0.2) (layer "F.Cu") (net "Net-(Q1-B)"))
 (segment (start 145.5 97.168629) (end 145.5 97.5) (width 0.2) (layer "F.Cu") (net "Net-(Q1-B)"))
 (segment (start 144.64038 96.640381) (end 145.499999 97.5) (width 0.2) (layer "F.Cu") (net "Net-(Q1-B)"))
 (segment (start 135 83.5) (end 144.64038 93.14038) (width 0.2) (layer "F.Cu") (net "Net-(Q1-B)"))
 (segment (start 123 83.5) (end 135 83.5) (width 0.2) (layer "F.Cu") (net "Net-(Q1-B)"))
 (segment (start 113.44 77.46) (end 118.94 77.46) (width 0.2) (layer "F.Cu") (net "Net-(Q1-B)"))
 (segment (start 176.03 78.72) (end 174.709208 78.72) (width 0.2) (layer "F.Cu") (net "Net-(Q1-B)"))
 (segment (start 120 80.5) (end 123 83.5) (width 0.2) (layer "F.Cu") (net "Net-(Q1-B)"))
 (segment (start 145.499999 97.5) (end 145.5 97.5) (width 0.2) (layer "F.Cu") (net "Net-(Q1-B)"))
 (segment (start 146.65 97.5) (end 145.5 97.5) (width 0.2) (layer "F.Cu") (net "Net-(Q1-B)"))
 (segment (start 176.5 78.25) (end 176.03 78.72) (width 0.2) (layer "F.Cu") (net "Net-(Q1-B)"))
 (segment (start 120 78.52) (end 120 80.5) (width 0.2) (layer "F.Cu") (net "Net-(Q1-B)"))
 (segment (start 146.05 96.45) (end 145.065075 96.45) (width 0.2) (layer "F.Cu") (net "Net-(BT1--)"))
 (segment (start 171.625 83.125) (end 161.725 83.125) (width 0.2) (layer "F.Cu") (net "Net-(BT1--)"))
 (segment (start 175.23 79.52) (end 171.625 83.125) (width 0.2) (layer "F.Cu") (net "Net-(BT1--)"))
 (segment (start 148.9 95.95) (end 148.9 97.5) (width 0.2) (layer "F.Cu") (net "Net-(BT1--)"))
 (segment (start 161.725 83.125) (end 148.9 95.95) (width 0.2) (layer "F.Cu") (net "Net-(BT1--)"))
 (segment (start 146.5 95.5) (end 146.5 96) (width 0.2) (layer "F.Cu") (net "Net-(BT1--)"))
 (segment (start 146.5 96) (end 146.05 96.45) (width 0.2) (layer "F.Cu") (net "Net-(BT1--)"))
 (via (at 146.5 95.5) (size 0.6) (drill 0.3) (layers "F.Cu" "B.Cu") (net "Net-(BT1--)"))
 (segment (start 148 98.4) (end 148.9 97.5) (width 0.2) (layer "B.Cu") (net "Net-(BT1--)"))
 (segment (start 148 114.5) (end 148 98.4) (width 0.2) (layer "B.Cu") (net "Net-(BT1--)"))
 (segment (start 146.5 95.5) (end 146.5 96.9) (width 0.2) (layer "B.Cu") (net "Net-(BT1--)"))
 (segment (start 146.5 96.9) (end 148 98.4) (width 0.2) (layer "B.Cu") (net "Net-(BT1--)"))
 (segment (start 177.77 79.52) (end 178 79.75) (width 0.2) (layer "F.Cu") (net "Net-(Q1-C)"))
 (segment (start 178 108) (end 156 130) (width 0.2) (layer "F.Cu") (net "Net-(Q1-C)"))
 (segment (start 156 130) (end 151.81 130) (width 0.2) (layer "F.Cu") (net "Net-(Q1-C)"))
 (segment (start 178 79.75) (end 178 108) (width 0.2) (layer "F.Cu") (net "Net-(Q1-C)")))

